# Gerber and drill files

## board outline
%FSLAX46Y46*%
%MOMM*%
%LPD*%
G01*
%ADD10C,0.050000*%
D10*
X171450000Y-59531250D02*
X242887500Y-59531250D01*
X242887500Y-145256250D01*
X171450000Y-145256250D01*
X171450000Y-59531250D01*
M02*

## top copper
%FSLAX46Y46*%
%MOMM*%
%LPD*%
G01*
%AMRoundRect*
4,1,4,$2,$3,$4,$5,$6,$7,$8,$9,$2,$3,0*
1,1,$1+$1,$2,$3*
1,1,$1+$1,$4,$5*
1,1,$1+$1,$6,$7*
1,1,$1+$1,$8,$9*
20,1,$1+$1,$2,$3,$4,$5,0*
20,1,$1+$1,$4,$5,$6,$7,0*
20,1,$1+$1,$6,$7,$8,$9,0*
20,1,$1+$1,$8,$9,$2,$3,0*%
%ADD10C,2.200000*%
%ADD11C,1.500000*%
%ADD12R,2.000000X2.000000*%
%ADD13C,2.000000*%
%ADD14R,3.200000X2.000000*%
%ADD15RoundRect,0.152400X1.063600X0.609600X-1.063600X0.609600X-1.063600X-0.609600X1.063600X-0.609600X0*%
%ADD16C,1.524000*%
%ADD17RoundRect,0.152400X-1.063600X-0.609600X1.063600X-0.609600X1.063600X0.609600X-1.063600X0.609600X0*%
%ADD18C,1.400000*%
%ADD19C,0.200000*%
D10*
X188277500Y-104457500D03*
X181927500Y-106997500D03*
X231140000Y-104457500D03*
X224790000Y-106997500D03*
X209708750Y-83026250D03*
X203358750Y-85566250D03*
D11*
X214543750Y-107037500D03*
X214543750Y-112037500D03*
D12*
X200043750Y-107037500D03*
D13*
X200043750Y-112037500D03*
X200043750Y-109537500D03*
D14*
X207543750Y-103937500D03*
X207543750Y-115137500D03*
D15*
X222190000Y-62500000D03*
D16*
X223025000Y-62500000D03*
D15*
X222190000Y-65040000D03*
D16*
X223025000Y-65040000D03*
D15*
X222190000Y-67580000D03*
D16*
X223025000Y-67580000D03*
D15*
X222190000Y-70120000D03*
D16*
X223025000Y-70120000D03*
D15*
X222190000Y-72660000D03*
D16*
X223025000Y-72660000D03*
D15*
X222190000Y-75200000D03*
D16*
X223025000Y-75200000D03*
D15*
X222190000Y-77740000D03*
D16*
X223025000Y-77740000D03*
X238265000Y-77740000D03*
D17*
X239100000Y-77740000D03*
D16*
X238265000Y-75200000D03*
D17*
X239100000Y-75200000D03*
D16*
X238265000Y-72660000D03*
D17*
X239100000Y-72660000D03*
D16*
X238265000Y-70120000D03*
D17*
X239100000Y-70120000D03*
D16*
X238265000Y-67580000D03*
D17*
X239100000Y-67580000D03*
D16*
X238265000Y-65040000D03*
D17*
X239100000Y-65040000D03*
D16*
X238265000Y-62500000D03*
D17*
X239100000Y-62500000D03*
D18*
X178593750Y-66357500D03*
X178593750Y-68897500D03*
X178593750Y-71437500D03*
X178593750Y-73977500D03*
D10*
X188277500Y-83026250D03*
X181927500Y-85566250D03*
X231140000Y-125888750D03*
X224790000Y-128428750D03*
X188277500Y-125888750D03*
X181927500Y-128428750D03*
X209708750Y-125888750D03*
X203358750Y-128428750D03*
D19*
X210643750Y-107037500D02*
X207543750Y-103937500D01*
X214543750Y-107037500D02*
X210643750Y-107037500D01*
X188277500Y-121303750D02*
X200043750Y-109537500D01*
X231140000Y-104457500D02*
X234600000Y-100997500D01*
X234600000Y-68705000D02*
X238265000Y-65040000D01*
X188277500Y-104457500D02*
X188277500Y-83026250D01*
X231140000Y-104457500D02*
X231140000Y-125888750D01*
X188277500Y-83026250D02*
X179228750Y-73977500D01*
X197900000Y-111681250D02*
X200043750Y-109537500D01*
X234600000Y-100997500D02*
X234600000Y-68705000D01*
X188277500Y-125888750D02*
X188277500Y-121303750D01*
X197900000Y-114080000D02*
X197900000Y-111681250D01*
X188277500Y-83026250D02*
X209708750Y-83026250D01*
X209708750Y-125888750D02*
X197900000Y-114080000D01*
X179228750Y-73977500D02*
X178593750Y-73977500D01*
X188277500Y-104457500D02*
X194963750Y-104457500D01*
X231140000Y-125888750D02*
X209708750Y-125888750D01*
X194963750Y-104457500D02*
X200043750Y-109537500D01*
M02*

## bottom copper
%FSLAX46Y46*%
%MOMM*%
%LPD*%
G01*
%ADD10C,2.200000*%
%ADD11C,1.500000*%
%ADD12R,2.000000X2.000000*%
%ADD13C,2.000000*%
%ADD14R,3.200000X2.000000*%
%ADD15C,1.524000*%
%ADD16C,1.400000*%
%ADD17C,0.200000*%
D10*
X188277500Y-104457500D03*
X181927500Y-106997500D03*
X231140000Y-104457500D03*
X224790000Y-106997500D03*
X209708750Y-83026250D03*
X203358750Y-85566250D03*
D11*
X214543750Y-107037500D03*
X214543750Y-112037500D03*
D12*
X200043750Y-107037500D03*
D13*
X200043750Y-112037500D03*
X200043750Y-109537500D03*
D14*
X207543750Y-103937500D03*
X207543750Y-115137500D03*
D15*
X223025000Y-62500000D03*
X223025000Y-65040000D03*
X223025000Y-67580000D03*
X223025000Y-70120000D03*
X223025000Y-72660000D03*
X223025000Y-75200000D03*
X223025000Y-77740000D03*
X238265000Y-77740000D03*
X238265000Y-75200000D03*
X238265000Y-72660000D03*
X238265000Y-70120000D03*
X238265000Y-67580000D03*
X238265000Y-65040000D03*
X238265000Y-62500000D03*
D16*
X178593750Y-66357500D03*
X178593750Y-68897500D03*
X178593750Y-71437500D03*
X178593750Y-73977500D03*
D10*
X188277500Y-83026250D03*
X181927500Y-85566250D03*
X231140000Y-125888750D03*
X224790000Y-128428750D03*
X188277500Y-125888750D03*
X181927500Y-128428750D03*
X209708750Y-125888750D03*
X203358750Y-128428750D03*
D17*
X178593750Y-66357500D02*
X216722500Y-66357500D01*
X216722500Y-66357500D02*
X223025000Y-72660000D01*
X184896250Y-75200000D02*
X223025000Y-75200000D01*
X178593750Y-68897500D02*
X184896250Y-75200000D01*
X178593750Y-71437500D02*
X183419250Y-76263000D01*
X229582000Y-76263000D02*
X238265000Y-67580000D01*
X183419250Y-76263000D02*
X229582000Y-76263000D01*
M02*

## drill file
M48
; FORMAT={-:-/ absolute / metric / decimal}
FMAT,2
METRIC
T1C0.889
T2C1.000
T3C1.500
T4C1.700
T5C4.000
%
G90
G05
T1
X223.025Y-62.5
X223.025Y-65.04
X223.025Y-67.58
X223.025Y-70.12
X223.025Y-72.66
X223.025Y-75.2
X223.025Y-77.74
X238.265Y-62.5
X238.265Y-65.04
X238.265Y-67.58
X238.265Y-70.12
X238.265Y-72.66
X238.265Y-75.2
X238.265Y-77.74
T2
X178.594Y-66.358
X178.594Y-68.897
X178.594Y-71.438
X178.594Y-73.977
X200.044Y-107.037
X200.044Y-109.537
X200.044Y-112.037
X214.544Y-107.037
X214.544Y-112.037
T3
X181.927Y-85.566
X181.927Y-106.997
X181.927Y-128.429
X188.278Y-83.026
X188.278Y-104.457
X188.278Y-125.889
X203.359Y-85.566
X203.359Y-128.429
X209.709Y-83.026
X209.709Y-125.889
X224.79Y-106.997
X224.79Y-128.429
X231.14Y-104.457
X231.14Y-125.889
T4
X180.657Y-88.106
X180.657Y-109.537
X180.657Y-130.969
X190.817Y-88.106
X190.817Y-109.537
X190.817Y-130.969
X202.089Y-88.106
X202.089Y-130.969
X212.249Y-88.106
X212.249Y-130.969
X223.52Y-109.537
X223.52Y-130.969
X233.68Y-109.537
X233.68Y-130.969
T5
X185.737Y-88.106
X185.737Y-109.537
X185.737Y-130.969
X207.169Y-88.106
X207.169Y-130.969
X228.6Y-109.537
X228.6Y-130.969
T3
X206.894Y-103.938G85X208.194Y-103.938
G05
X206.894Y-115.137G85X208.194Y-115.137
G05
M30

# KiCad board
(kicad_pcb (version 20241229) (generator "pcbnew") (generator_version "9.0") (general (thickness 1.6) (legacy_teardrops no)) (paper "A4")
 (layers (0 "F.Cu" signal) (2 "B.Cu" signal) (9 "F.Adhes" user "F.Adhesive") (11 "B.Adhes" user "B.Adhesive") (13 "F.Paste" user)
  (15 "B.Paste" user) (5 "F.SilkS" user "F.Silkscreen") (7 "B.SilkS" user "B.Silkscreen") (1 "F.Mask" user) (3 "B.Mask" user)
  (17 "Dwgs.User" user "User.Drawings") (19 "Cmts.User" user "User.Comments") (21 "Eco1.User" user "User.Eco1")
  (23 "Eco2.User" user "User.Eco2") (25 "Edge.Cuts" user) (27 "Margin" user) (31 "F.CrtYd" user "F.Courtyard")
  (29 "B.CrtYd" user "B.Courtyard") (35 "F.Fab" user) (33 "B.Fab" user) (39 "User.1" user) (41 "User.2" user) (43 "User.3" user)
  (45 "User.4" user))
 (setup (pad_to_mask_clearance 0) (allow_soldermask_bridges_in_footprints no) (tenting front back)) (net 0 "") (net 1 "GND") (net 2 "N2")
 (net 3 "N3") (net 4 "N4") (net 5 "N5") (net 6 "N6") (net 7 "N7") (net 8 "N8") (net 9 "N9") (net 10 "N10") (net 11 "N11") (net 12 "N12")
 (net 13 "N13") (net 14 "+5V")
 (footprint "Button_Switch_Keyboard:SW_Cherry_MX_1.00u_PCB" (layer "F.Cu") (at 188.2775 104.4575)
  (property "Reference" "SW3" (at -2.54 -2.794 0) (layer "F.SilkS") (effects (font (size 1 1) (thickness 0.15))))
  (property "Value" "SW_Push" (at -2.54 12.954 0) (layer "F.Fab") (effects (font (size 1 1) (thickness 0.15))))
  (pad "" np_thru_hole circle (at -7.62 5.08) (size 1.7 1.7) (drill 1.7) (layers "*.Cu" "*.Mask"))
  (pad "" np_thru_hole circle (at -2.54 5.08) (size 4 4) (drill 4) (layers "*.Cu" "*.Mask"))
  (pad "" np_thru_hole circle (at 2.54 5.08) (size 1.7 1.7) (drill 1.7) (layers "*.Cu" "*.Mask"))
  (pad "1" thru_hole circle (at 0 0) (size 2.2 2.2) (drill 1.5) (layers "*.Cu" "*.Mask") (remove_unused_layers no) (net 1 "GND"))
  (pad "2" thru_hole circle (at -6.35 2.54) (size 2.2 2.2) (drill 1.5) (layers "*.Cu" "*.Mask") (remove_unused_layers no) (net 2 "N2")))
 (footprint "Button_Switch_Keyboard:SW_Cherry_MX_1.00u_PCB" (layer "F.Cu") (at 231.14 104.4575)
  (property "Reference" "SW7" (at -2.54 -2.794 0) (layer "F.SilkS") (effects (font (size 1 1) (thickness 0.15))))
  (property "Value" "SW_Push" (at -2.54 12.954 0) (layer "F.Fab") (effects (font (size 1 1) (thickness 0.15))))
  (pad "" np_thru_hole circle (at -7.62 5.08) (size 1.7 1.7) (drill 1.7) (layers "*.Cu" "*.Mask"))
  (pad "" np_thru_hole circle (at -2.54 5.08) (size 4 4) (drill 4) (layers "*.Cu" "*.Mask"))
  (pad "" np_thru_hole circle (at 2.54 5.08) (size 1.7 1.7) (drill 1.7) (layers "*.Cu" "*.Mask"))
  (pad "1" thru_hole circle (at 0 0) (size 2.2 2.2) (drill 1.5) (layers "*.Cu" "*.Mask") (remove_unused_layers no) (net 1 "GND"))
  (pad "2" thru_hole circle (at -6.35 2.54) (size 2.2 2.2) (drill 1.5) (layers "*.Cu" "*.Mask") (remove_unused_layers no) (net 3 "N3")))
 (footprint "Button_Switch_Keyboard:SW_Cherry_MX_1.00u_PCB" (layer "F.Cu") (at 209.70875 83.02625)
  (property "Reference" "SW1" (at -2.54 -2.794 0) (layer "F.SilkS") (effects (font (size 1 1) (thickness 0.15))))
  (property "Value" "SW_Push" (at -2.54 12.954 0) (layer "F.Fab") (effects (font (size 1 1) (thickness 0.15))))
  (pad "" np_thru_hole circle (at -7.62 5.08) (size 1.7 1.7) (drill 1.7) (layers "*.Cu" "*.Mask"))
  (pad "" np_thru_hole circle (at -2.54 5.08) (size 4 4) (drill 4) (layers "*.Cu" "*.Mask"))
  (pad "" np_thru_hole circle (at 2.54 5.08) (size 1.7 1.7) (drill 1.7) (layers "*.Cu" "*.Mask"))
  (pad "1" thru_hole circle (at 0 0) (size 2.2 2.2) (drill 1.5) (layers "*.Cu" "*.Mask") (remove_unused_layers no) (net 1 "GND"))
  (pad "2" thru_hole circle (at -6.35 2.54) (size 2.2 2.2) (drill 1.5) (layers "*.Cu" "*.Mask") (remove_unused_layers no) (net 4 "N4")))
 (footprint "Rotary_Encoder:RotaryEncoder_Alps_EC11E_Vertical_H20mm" (layer "F.Cu") (at 200.04375 107.0375)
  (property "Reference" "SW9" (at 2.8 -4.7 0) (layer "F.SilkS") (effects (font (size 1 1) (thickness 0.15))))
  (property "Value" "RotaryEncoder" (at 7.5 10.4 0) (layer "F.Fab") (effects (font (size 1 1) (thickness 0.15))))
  (pad "" thru_hole circle (at 14.5 0) (size 1.5 1.5) (drill 1) (layers "*.Cu" "*.Mask") (remove_unused_layers no))
  (pad "" thru_hole circle (at 14.5 5) (size 1.5 1.5) (drill 1) (layers "*.Cu" "*.Mask") (remove_unused_layers no))
  (pad "A" thru_hole rect (at 0 0) (size 2 2) (drill 1) (layers "*.Cu" "*.Mask") (remove_unused_layers no) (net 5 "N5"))
  (pad "B" thru_hole circle (at 0 5) (size 2 2) (drill 1) (layers "*.Cu" "*.Mask") (remove_unused_layers no) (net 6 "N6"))
  (pad "C" thru_hole circle (at 0 2.5) (size 2 2) (drill 1) (layers "*.Cu" "*.Mask") (remove_unused_layers no) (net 1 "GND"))
  (pad "MP" thru_hole rect (at 7.5 -3.1) (size 3.2 2) (drill oval 2.8 1.5) (layers "*.Cu" "*.Mask") (remove_unused_layers no))
  (pad "MP" thru_hole rect (at 7.5 8.1) (size 3.2 2) (drill oval 2.8 1.5) (layers "*.Cu" "*.Mask") (remove_unused_layers no)))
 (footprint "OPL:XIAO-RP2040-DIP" (layer "F.Cu") (at 230.645 70.12)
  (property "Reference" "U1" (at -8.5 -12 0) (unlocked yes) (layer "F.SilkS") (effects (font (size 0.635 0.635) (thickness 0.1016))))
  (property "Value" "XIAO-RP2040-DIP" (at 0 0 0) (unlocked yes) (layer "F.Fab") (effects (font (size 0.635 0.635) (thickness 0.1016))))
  (pad "1" smd roundrect (at -8.455 -7.62 180) (size 2.432 1.524) (layers "F.Cu" "F.Mask") (roundrect_rratio 0.1) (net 4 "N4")
   (thermal_bridge_angle 45))
  (pad "1" thru_hole circle (at -7.62 -7.62 180) (size 1.524 1.524) (drill 0.889) (layers "*.Cu" "*.Mask") (remove_unused_layers no)
   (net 4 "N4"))
  (pad "2" smd roundrect (at -8.455 -5.08 180) (size 2.432 1.524) (layers "F.Cu" "F.Mask") (roundrect_rratio 0.1) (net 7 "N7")
   (thermal_bridge_angle 45))
  (pad "2" thru_hole circle (at -7.62 -5.08 180) (size 1.524 1.524) (drill 0.889) (layers "*.Cu" "*.Mask") (remove_unused_layers no)
   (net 7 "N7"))
  (pad "3" smd roundrect (at -8.455 -2.54 180) (size 2.432 1.524) (layers "F.Cu" "F.Mask") (roundrect_rratio 0.1) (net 2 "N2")
   (thermal_bridge_angle 45))
  (pad "3" thru_hole circle (at -7.62 -2.54 180) (size 1.524 1.524) (drill 0.889) (layers "*.Cu" "*.Mask") (remove_unused_layers no)
   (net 2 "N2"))
  (pad "4" smd roundrect (at -8.455 0 180) (size 2.432 1.524) (layers "F.Cu" "F.Mask") (roundrect_rratio 0.1) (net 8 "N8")
   (thermal_bridge_angle 45))
  (pad "4" thru_hole circle (at -7.62 0 180) (size 1.524 1.524) (drill 0.889) (layers "*.Cu" "*.Mask") (remove_unused_layers no)
   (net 8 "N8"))
  (pad "5" smd roundrect (at -8.455 2.54 180) (size 2.432 1.524) (layers "F.Cu" "F.Mask") (roundrect_rratio 0.1) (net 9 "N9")
   (thermal_bridge_angle 45))
  (pad "5" thru_hole circle (at -7.62 2.54 180) (size 1.524 1.524) (drill 0.889) (layers "*.Cu" "*.Mask") (remove_unused_layers no)
   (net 9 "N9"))
  (pad "6" smd roundrect (at -8.455 5.08 180) (size 2.432 1.524) (layers "F.Cu" "F.Mask") (roundrect_rratio 0.1) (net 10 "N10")
   (thermal_bridge_angle 45))
  (pad "6" thru_hole circle (at -7.62 5.08 180) (size 1.524 1.524) (drill 0.889) (layers "*.Cu" "*.Mask") (remove_unused_layers no)
   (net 10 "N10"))
  (pad "7" smd roundrect (at -8.455 7.62 180) (size 2.432 1.524) (layers "F.Cu" "F.Mask") (roundrect_rratio 0.1) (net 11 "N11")
   (thermal_bridge_angle 45))
  (pad "7" thru_hole circle (at -7.62 7.62 180) (size 1.524 1.524) (drill 0.889) (layers "*.Cu" "*.Mask") (remove_unused_layers no)
   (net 11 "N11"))
  (pad "8" thru_hole circle (at 7.62 7.62) (size 1.524 1.524) (drill 0.889) (layers "*.Cu" "*.Mask") (remove_unused_layers no)
   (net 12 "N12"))
  (pad "8" smd roundrect (at 8.455 7.62) (size 2.432 1.524) (layers "F.Cu" "F.Mask") (roundrect_rratio 0.1) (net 12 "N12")
   (thermal_bridge_angle 45))
  (pad "9" thru_hole circle (at 7.62 5.08) (size 1.524 1.524) (drill 0.889) (layers "*.Cu" "*.Mask") (remove_unused_layers no) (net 3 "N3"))
  (pad "9" smd roundrect (at 8.455 5.08) (size 2.432 1.524) (layers "F.Cu" "F.Mask") (roundrect_rratio 0.1) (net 3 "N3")
   (thermal_bridge_angle 45))
  (pad "10" thru_hole circle (at 7.62 2.54) (size 1.524 1.524) (drill 0.889) (layers "*.Cu" "*.Mask") (remove_unused_layers no) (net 6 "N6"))
  (pad "10" smd roundrect (at 8.455 2.54) (size 2.432 1.524) (layers "F.Cu" "F.Mask") (roundrect_rratio 0.1) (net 6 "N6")
   (thermal_bridge_angle 45))
  (pad "11" thru_hole circle (at 7.62 0) (size 1.524 1.524) (drill 0.889) (layers "*.Cu" "*.Mask") (remove_unused_layers no) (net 5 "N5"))
  (pad "11" smd roundrect (at 8.455 0) (size 2.432 1.524) (layers "F.Cu" "F.Mask") (roundrect_rratio 0.1) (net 5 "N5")
   (thermal_bridge_angle 45))
  (pad "12" thru_hole circle (at 7.62 -2.54) (size 1.524 1.524) (drill 0.889) (layers "*.Cu" "*.Mask") (remove_unused_layers no)
   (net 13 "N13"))
  (pad "12" smd roundrect (at 8.455 -2.54) (size 2.432 1.524) (layers "F.Cu" "F.Mask") (roundrect_rratio 0.1) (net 13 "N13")
   (thermal_bridge_angle 45))
  (pad "13" thru_hole circle (at 7.62 -5.08) (size 1.524 1.524) (drill 0.889) (layers "*.Cu" "*.Mask") (remove_unused_layers no)
   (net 1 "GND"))
  (pad "13" smd roundrect (at 8.455 -5.08) (size 2.432 1.524) (layers "F.Cu" "F.Mask") (roundrect_rratio 0.1) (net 1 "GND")
   (thermal_bridge_angle 45))
  (pad "14" thru_hole circle (at 7.62 -7.62) (size 1.524 1.524) (drill 0.889) (layers "*.Cu" "*.Mask") (remove_unused_layers no)
   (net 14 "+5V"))
  (pad "14" smd roundrect (at 8.455 -7.62) (size 2.432 1.524) (layers "F.Cu" "F.Mask") (roundrect_rratio 0.1) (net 14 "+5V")
   (thermal_bridge_angle 45)))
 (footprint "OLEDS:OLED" (layer "F.Cu") (at 178.59375 70.1675 -90)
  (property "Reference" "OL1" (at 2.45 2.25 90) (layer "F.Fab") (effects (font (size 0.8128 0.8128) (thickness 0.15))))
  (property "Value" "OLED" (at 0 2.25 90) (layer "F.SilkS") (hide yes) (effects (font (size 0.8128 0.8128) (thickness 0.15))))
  (pad "1" thru_hole circle (at -3.81 0 270) (size 1.4 1.4) (drill 1) (layers "*.Cu" "*.Mask") (remove_unused_layers no) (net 9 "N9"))
  (pad "2" thru_hole circle (at -1.27 0 270) (size 1.4 1.4) (drill 1) (layers "*.Cu" "*.Mask") (remove_unused_layers no) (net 10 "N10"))
  (pad "3" thru_hole circle (at 1.27 0 270) (size 1.4 1.4) (drill 1) (layers "*.Cu" "*.Mask") (remove_unused_layers no) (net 13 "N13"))
  (pad "4" thru_hole circle (at 3.81 0 270) (size 1.4 1.4) (drill 1) (layers "*.Cu" "*.Mask") (remove_unused_layers no) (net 1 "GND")))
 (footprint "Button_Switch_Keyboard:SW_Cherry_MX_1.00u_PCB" (layer "F.Cu") (at 188.2775 83.02625)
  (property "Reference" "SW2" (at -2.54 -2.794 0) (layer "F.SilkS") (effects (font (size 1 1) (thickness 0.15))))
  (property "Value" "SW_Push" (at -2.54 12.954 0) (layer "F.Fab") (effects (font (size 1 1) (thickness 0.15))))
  (pad "" np_thru_hole circle (at -7.62 5.08) (size 1.7 1.7) (drill 1.7) (layers "*.Cu" "*.Mask"))
  (pad "" np_thru_hole circle (at -2.54 5.08) (size 4 4) (drill 4) (layers "*.Cu" "*.Mask"))
  (pad "" np_thru_hole circle (at 2.54 5.08) (size 1.7 1.7) (drill 1.7) (layers "*.Cu" "*.Mask"))
  (pad "1" thru_hole circle (at 0 0) (size 2.2 2.2) (drill 1.5) (layers "*.Cu" "*.Mask") (remove_unused_layers no) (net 1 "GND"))
  (pad "2" thru_hole circle (at -6.35 2.54) (size 2.2 2.2) (drill 1.5) (layers "*.Cu" "*.Mask") (remove_unused_layers no) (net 7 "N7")))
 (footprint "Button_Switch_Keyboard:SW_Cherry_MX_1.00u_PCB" (layer "F.Cu") (at 231.14 125.88875)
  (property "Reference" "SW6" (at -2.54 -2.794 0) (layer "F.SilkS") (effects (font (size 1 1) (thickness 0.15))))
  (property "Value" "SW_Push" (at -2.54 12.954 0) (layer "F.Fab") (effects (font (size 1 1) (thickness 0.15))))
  (pad "" np_thru_hole circle (at -7.62 5.08) (size 1.7 1.7) (drill 1.7) (layers "*.Cu" "*.Mask"))
  (pad "" np_thru_hole circle (at -2.54 5.08) (size 4 4) (drill 4) (layers "*.Cu" "*.Mask"))
  (pad "" np_thru_hole circle (at 2.54 5.08) (size 1.7 1.7) (drill 1.7) (layers "*.Cu" "*.Mask"))
  (pad "1" thru_hole circle (at 0 0) (size 2.2 2.2) (drill 1.5) (layers "*.Cu" "*.Mask") (remove_unused_layers no) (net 1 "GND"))
  (pad "2" thru_hole circle (at -6.35 2.54) (size 2.2 2.2) (drill 1.5) (layers "*.Cu" "*.Mask") (remove_unused_layers no) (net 12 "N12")))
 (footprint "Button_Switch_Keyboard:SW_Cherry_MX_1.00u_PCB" (layer "F.Cu") (at 188.2775 125.88875)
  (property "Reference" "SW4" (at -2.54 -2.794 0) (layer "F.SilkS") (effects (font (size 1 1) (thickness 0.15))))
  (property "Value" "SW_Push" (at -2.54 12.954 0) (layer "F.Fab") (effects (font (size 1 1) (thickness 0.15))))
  (pad "" np_thru_hole circle (at -7.62 5.08) (size 1.7 1.7) (drill 1.7) (layers "*.Cu" "*.Mask"))
  (pad "" np_thru_hole circle (at -2.54 5.08) (size 4 4) (drill 4) (layers "*.Cu" "*.Mask"))
  (pad "" np_thru_hole circle (at 2.54 5.08) (size 1.7 1.7) (drill 1.7) (layers "*.Cu" "*.Mask"))
  (pad "1" thru_hole circle (at 0 0) (size 2.2 2.2) (drill 1.5) (layers "*.Cu" "*.Mask") (remove_unused_layers no) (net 1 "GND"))
  (pad "2" thru_hole circle (at -6.35 2.54) (size 2.2 2.2) (drill 1.5) (layers "*.Cu" "*.Mask") (remove_unused_layers no) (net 8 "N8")))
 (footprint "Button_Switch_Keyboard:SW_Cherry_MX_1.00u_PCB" (layer "F.Cu") (at 209.70875 125.88875)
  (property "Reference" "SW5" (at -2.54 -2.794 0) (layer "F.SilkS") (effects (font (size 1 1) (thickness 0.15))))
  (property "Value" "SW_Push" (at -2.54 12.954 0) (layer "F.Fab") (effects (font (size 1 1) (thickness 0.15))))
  (pad "" np_thru_hole circle (at -7.62 5.08) (size 1.7 1.7) (drill 1.7) (layers "*.Cu" "*.Mask"))
  (pad "" np_thru_hole circle (at -2.54 5.08) (size 4 4) (drill 4) (layers "*.Cu" "*.Mask"))
  (pad "" np_thru_hole circle (at 2.54 5.08) (size 1.7 1.7) (drill 1.7) (layers "*.Cu" "*.Mask"))
  (pad "1" thru_hole circle (at 0 0) (size 2.2 2.2) (drill 1.5) (layers "*.Cu" "*.Mask") (remove_unused_layers no) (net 1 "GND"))
  (pad "2" thru_hole circle (at -6.35 2.54) (size 2.2 2.2) (drill 1.5) (layers "*.Cu" "*.Mask") (remove_unused_layers no) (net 11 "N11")))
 (gr_rect (start 171.45 59.53125) (end 242.8875 145.25625) (stroke (width 0.05) (type default)) (fill no) (layer "Edge.Cuts"))
 (segment (start 210.64375 107.0375) (end 207.54375 103.9375) (width 0.2) (layer "F.Cu") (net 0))
 (segment (start 214.54375 107.0375) (end 210.64375 107.0375) (width 0.2) (layer "F.Cu") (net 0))
 (segment (start 178.59375 66.3575) (end 216.7225 66.3575) (width 0.2) (layer "B.Cu") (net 9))
 (segment (start 216.7225 66.3575) (end 223.025 72.66) (width 0.2) (layer "B.Cu") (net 9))
 (segment (start 184.89625 75.2) (end 223.025 75.2) (width 0.2) (layer "B.Cu") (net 10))
 (segment (start 178.59375 68.8975) (end 184.89625 75.2) (width 0.2) (layer "B.Cu") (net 10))
 (segment (start 178.59375 71.4375) (end 183.41925 76.263) (width 0.2) (layer "B.Cu") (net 13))
 (segment (start 229.582 76.263) (end 238.265 67.58) (width 0.2) (layer "B.Cu") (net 13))
 (segment (start 183.41925 76.263) (end 229.582 76.263) (width 0.2) (layer "B.Cu") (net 13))
 (segment (start 188.2775 121.30375) (end 200.04375 109.5375) (width 0.2) (layer "F.Cu") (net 1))
 (segment (start 231.14 104.4575) (end 234.6 100.9975) (width 0.2) (layer "F.Cu") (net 1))
 (segment (start 234.6 68.705) (end 238.265 65.04) (width 0.2) (layer "F.Cu") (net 1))
 (segment (start 188.2775 104.4575) (end 188.2775 83.02625) (width 0.2) (layer "F.Cu") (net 1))
 (segment (start 231.14 104.4575) (end 231.14 125.88875) (width 0.2) (layer "F.Cu") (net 1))
 (segment (start 188.2775 83.02625) (end 179.22875 73.9775) (width 0.2) (layer "F.Cu") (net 1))
 (segment (start 197.9 111.68125) (end 200.04375 109.5375) (width 0.2) (layer "F.Cu") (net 1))
 (segment (start 234.6 100.9975) (end 234.6 68.705) (width 0.2) (layer "F.Cu") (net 1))
 (segment (start 188.2775 125.88875) (end 188.2775 121.30375) (width 0.2) (layer "F.Cu") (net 1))
 (segment (start 197.9 114.08) (end 197.9 111.68125) (width 0.2) (layer "F.Cu") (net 1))
 (segment (start 188.2775 83.02625) (end 209.70875 83.02625) (width 0.2) (layer "F.Cu") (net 1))
 (segment (start 209.70875 125.88875) (end 197.9 114.08) (width 0.2) (layer "F.Cu") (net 1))
 (segment (start 179.22875 73.9775) (end 178.59375 73.9775) (width 0.2) (layer "F.Cu") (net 1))
 (segment (start 188.2775 104.4575) (end 194.96375 104.4575) (width 0.2) (layer "F.Cu") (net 1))
 (segment (start 231.14 125.88875) (end 209.70875 125.88875) (width 0.2) (layer "F.Cu") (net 1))
 (segment (start 194.96375 104.4575) (end 200.04375 109.5375) (width 0.2) (layer "F.Cu") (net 1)))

